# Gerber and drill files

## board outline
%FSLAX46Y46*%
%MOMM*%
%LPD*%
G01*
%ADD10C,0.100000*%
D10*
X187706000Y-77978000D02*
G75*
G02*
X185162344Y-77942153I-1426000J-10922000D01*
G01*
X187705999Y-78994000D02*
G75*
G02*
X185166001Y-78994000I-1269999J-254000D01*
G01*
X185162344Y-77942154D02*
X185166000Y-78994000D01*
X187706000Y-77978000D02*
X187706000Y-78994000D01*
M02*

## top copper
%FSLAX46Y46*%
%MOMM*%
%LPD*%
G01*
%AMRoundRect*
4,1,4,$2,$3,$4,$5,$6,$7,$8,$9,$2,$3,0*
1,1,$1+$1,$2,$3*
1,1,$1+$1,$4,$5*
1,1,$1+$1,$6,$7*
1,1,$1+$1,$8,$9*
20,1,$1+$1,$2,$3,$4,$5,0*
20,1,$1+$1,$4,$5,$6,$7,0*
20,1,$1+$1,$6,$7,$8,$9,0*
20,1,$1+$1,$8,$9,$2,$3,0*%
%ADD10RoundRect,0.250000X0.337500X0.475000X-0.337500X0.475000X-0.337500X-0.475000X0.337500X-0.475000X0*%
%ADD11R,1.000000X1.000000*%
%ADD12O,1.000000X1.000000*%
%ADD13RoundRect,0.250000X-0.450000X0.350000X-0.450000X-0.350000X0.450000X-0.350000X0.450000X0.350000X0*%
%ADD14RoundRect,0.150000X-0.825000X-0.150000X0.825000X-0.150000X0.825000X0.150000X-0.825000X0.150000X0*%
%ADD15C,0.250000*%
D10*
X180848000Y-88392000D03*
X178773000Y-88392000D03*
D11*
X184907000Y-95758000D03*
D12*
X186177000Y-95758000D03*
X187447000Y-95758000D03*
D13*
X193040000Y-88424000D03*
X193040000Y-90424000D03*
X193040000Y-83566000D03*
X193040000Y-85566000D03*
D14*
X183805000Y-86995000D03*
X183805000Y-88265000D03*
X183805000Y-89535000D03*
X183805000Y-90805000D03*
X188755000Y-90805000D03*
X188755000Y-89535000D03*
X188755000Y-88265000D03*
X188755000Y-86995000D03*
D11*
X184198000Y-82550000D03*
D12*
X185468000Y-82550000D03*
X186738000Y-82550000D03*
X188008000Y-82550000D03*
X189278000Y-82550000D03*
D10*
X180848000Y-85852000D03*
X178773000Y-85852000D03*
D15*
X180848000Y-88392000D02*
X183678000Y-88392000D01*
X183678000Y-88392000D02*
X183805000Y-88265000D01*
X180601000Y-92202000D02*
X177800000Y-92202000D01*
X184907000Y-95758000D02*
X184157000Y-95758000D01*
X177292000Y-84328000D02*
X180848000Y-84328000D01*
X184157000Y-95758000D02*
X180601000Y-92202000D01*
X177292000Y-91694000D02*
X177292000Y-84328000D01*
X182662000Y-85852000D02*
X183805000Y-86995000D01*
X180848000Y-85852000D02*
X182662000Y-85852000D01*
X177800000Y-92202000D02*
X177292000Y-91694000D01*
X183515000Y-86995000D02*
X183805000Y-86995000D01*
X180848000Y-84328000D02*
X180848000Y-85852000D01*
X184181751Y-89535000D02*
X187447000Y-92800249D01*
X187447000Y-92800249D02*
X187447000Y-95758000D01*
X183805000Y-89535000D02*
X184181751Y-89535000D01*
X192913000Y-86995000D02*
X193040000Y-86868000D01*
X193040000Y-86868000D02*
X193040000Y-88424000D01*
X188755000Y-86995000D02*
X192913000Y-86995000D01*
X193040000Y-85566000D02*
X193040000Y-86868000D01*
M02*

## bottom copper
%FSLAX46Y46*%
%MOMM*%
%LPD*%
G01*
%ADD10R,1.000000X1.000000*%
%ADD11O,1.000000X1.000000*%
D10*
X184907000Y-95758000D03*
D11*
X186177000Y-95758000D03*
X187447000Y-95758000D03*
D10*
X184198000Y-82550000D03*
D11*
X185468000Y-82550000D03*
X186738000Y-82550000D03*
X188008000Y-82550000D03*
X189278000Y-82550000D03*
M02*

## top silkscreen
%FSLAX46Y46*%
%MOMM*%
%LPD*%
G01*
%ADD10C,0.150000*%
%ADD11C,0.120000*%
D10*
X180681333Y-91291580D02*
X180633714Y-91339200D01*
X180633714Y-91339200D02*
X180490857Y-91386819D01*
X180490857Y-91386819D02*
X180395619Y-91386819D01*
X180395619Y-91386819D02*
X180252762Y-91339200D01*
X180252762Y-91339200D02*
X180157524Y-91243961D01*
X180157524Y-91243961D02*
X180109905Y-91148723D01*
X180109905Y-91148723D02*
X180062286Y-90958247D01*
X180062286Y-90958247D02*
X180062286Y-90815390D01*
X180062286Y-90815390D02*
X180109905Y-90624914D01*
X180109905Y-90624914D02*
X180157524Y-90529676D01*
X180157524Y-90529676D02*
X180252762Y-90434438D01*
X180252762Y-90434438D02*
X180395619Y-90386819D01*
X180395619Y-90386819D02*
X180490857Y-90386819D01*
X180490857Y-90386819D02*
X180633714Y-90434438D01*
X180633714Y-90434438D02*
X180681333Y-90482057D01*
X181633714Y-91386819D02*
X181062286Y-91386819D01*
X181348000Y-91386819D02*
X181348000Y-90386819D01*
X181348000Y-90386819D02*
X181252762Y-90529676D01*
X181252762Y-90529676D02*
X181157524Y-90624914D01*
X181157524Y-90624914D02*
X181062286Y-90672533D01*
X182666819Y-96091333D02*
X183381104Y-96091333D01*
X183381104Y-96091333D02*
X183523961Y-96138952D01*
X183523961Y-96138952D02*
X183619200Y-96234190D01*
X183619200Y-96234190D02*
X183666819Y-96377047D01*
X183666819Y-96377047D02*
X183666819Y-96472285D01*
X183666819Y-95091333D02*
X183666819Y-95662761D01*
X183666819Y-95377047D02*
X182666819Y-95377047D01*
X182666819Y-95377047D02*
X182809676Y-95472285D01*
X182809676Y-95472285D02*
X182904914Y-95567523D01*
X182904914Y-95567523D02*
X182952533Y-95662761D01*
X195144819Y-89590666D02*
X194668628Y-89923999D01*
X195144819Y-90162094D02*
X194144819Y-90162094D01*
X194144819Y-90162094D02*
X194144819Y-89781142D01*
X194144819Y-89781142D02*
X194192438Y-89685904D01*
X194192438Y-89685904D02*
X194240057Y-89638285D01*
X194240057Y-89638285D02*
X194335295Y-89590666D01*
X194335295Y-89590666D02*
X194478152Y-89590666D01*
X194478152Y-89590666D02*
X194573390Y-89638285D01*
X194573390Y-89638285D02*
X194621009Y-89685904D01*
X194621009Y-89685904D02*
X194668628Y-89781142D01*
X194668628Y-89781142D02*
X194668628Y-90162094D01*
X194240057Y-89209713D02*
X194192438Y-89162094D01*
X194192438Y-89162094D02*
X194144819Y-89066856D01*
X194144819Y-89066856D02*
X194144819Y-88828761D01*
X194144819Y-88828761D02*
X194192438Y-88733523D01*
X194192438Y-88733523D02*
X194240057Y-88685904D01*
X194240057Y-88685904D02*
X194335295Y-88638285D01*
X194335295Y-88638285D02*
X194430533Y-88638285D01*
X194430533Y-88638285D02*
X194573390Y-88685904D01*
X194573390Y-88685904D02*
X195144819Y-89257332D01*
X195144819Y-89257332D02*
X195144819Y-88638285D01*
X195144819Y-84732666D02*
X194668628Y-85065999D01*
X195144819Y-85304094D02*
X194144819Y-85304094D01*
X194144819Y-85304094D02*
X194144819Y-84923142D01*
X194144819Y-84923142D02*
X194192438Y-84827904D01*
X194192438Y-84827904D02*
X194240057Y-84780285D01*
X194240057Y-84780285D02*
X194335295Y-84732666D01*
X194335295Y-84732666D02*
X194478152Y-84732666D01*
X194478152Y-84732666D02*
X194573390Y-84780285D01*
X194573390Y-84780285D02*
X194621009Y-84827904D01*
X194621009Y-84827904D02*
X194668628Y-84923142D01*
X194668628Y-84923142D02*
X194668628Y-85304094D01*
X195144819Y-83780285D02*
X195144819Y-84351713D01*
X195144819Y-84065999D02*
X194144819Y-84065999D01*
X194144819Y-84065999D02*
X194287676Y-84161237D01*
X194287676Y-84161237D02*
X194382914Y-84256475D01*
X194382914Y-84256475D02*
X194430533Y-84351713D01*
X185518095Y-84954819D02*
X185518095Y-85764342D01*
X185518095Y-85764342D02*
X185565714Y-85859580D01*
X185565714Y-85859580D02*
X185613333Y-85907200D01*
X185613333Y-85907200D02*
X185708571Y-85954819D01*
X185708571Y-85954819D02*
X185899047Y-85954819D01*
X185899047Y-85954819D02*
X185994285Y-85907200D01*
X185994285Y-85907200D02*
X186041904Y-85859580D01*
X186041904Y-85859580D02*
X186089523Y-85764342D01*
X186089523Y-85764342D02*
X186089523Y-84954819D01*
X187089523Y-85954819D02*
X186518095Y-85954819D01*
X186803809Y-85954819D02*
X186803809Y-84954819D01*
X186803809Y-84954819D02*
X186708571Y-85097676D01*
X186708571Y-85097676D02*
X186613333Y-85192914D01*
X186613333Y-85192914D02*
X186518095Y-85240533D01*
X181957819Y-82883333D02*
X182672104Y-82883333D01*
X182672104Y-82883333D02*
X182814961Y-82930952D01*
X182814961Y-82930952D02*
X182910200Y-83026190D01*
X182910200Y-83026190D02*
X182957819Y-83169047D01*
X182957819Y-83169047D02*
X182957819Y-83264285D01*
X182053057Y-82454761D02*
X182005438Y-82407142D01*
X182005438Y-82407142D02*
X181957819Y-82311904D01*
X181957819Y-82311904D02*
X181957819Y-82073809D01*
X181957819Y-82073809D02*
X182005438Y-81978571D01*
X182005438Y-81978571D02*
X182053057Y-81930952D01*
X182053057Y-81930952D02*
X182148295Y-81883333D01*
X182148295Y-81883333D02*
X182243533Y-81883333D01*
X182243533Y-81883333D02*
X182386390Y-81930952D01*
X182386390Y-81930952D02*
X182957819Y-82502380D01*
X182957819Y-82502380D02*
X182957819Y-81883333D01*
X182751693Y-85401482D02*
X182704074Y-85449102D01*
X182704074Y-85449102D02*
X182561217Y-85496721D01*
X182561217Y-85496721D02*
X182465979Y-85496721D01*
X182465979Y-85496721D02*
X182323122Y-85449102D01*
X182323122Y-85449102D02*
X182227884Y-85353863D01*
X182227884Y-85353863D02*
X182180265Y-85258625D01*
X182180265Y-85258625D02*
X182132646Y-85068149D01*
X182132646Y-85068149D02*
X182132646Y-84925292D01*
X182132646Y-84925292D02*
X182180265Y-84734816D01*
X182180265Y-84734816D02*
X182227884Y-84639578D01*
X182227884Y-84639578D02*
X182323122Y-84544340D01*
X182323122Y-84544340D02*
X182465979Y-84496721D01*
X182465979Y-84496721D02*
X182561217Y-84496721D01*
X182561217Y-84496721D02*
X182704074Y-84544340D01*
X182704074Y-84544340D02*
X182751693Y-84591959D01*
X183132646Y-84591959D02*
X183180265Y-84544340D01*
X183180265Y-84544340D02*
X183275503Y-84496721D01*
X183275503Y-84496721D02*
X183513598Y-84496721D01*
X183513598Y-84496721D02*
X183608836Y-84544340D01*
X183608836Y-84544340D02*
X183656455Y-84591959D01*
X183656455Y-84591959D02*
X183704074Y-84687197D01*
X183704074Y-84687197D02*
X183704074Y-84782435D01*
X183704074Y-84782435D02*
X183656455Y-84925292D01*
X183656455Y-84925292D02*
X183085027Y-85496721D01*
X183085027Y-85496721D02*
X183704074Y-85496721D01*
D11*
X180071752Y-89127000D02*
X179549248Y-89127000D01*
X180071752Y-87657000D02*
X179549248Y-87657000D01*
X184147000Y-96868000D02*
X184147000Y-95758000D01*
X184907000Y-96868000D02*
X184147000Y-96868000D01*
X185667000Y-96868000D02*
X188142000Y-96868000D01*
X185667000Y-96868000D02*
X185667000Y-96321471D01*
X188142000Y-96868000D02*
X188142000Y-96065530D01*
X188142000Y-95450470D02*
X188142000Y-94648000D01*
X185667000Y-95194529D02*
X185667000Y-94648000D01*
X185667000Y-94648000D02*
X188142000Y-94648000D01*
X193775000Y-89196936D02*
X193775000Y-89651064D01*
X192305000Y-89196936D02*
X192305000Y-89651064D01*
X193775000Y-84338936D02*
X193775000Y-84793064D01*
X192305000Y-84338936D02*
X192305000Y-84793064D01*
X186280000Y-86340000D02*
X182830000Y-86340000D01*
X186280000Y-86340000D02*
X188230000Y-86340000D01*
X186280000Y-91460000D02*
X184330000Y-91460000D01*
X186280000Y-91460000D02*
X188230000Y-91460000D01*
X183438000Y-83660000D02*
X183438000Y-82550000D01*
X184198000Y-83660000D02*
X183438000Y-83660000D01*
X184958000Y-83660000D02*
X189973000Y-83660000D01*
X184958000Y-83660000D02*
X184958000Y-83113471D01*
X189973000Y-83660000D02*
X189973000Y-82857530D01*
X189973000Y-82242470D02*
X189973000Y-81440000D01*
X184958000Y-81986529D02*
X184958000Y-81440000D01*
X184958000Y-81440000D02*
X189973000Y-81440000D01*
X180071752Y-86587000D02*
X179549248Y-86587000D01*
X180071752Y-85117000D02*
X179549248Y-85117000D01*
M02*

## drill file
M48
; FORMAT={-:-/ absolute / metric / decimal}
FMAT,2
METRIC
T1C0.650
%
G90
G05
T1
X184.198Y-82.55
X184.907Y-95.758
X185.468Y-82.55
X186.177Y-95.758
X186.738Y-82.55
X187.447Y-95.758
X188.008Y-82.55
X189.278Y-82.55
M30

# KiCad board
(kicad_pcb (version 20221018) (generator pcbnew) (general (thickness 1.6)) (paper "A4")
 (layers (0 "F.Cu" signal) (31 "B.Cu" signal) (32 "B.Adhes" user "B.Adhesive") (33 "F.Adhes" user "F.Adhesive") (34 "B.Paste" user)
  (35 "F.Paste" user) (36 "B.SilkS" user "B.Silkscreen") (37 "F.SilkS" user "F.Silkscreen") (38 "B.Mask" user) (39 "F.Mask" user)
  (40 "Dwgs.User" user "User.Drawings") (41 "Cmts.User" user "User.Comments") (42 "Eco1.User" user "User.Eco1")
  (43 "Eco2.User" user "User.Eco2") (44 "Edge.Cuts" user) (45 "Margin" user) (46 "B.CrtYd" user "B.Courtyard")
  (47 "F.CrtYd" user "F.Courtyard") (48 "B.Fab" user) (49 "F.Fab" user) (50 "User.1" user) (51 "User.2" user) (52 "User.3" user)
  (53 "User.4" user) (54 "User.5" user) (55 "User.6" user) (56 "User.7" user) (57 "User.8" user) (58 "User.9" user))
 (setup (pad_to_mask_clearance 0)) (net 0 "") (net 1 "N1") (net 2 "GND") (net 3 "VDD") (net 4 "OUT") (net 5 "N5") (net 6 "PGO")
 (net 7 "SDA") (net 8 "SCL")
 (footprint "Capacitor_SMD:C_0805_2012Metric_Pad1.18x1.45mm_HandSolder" (layer "F.Cu") (at 179.8105 88.392 180)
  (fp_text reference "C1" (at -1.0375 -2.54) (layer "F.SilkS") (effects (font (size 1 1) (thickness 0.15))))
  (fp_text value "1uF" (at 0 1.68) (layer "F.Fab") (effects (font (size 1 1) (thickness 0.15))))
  (fp_line (start -0.261252 -0.735) (end 0.261252 -0.735) (stroke (width 0.12) (type solid)) (layer "F.SilkS"))
  (fp_line (start -0.261252 0.735) (end 0.261252 0.735) (stroke (width 0.12) (type solid)) (layer "F.SilkS"))
  (pad "1" smd roundrect (at -1.0375 0 180) (size 1.175 1.45) (layers "F.Cu" "F.Paste" "F.Mask") (roundrect_rratio 0.212766) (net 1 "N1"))
  (pad "2" smd roundrect (at 1.0375 0 180) (size 1.175 1.45) (layers "F.Cu" "F.Paste" "F.Mask") (roundrect_rratio 0.212766) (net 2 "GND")))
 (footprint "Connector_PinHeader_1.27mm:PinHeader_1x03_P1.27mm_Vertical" (layer "F.Cu") (at 184.907 95.758 90)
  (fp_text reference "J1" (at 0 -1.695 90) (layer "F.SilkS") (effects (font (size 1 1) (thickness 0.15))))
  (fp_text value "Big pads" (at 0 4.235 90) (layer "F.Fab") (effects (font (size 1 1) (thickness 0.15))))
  (fp_line (start -1.11 -0.76) (end 0 -0.76) (stroke (width 0.12) (type solid)) (layer "F.SilkS"))
  (fp_line (start -1.11 0) (end -1.11 -0.76) (stroke (width 0.12) (type solid)) (layer "F.SilkS"))
  (fp_line (start -1.11 0.76) (end -1.11 3.235) (stroke (width 0.12) (type solid)) (layer "F.SilkS"))
  (fp_line (start -1.11 0.76) (end -0.563471 0.76) (stroke (width 0.12) (type solid)) (layer "F.SilkS"))
  (fp_line (start -1.11 3.235) (end -0.30753 3.235) (stroke (width 0.12) (type solid)) (layer "F.SilkS"))
  (fp_line (start 0.30753 3.235) (end 1.11 3.235) (stroke (width 0.12) (type solid)) (layer "F.SilkS"))
  (fp_line (start 0.563471 0.76) (end 1.11 0.76) (stroke (width 0.12) (type solid)) (layer "F.SilkS"))
  (fp_line (start 1.11 0.76) (end 1.11 3.235) (stroke (width 0.12) (type solid)) (layer "F.SilkS"))
  (pad "1" thru_hole rect (at 0 0 90) (size 1 1) (drill 0.65) (layers "*.Cu" "*.Mask") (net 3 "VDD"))
  (pad "2" thru_hole oval (at 0 1.27 90) (size 1 1) (drill 0.65) (layers "*.Cu" "*.Mask") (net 2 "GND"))
  (pad "3" thru_hole oval (at 0 2.54 90) (size 1 1) (drill 0.65) (layers "*.Cu" "*.Mask") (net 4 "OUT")))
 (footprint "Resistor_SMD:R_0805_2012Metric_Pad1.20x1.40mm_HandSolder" (layer "F.Cu") (at 193.04 89.424 -90)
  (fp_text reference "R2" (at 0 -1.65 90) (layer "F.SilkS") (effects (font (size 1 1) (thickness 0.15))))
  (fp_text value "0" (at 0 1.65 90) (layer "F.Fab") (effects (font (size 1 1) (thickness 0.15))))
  (fp_line (start -0.227064 -0.735) (end 0.227064 -0.735) (stroke (width 0.12) (type solid)) (layer "F.SilkS"))
  (fp_line (start -0.227064 0.735) (end 0.227064 0.735) (stroke (width 0.12) (type solid)) (layer "F.SilkS"))
  (pad "1" smd roundrect (at -1 0 270) (size 1.2 1.4) (layers "F.Cu" "F.Paste" "F.Mask") (roundrect_rratio 0.208333) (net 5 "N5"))
  (pad "2" smd roundrect (at 1 0 270) (size 1.2 1.4) (layers "F.Cu" "F.Paste" "F.Mask") (roundrect_rratio 0.208333) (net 2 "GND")))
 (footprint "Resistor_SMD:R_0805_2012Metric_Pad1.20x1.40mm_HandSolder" (layer "F.Cu") (at 193.04 84.566 -90)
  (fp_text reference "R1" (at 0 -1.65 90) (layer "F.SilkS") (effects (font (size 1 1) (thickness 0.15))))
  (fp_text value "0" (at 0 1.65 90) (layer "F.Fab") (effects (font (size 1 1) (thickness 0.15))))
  (fp_line (start -0.227064 -0.735) (end 0.227064 -0.735) (stroke (width 0.12) (type solid)) (layer "F.SilkS"))
  (fp_line (start -0.227064 0.735) (end 0.227064 0.735) (stroke (width 0.12) (type solid)) (layer "F.SilkS"))
  (pad "1" smd roundrect (at -1 0 270) (size 1.2 1.4) (layers "F.Cu" "F.Paste" "F.Mask") (roundrect_rratio 0.208333) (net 3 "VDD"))
  (pad "2" smd roundrect (at 1 0 270) (size 1.2 1.4) (layers "F.Cu" "F.Paste" "F.Mask") (roundrect_rratio 0.208333) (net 5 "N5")))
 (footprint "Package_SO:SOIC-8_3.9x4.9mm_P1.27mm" (layer "F.Cu") (at 186.28 88.9)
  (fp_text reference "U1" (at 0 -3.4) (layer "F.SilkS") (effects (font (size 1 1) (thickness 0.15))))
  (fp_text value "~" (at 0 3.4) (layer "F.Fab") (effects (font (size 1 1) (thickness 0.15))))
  (fp_line (start 0 -2.56) (end -3.45 -2.56) (stroke (width 0.12) (type solid)) (layer "F.SilkS"))
  (fp_line (start 0 -2.56) (end 1.95 -2.56) (stroke (width 0.12) (type solid)) (layer "F.SilkS"))
  (fp_line (start 0 2.56) (end -1.95 2.56) (stroke (width 0.12) (type solid)) (layer "F.SilkS"))
  (fp_line (start 0 2.56) (end 1.95 2.56) (stroke (width 0.12) (type solid)) (layer "F.SilkS"))
  (pad "1" smd roundrect (at -2.475 -1.905) (size 1.95 0.6) (layers "F.Cu" "F.Paste" "F.Mask") (roundrect_rratio 0.25) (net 3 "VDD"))
  (pad "2" smd roundrect (at -2.475 -0.635) (size 1.95 0.6) (layers "F.Cu" "F.Paste" "F.Mask") (roundrect_rratio 0.25) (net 1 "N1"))
  (pad "3" smd roundrect (at -2.475 0.635) (size 1.95 0.6) (layers "F.Cu" "F.Paste" "F.Mask") (roundrect_rratio 0.25) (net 4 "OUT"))
  (pad "4" smd roundrect (at -2.475 1.905) (size 1.95 0.6) (layers "F.Cu" "F.Paste" "F.Mask") (roundrect_rratio 0.25) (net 2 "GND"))
  (pad "5" smd roundrect (at 2.475 1.905) (size 1.95 0.6) (layers "F.Cu" "F.Paste" "F.Mask") (roundrect_rratio 0.25) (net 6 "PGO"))
  (pad "6" smd roundrect (at 2.475 0.635) (size 1.95 0.6) (layers "F.Cu" "F.Paste" "F.Mask") (roundrect_rratio 0.25) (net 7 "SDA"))
  (pad "7" smd roundrect (at 2.475 -0.635) (size 1.95 0.6) (layers "F.Cu" "F.Paste" "F.Mask") (roundrect_rratio 0.25) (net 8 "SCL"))
  (pad "8" smd roundrect (at 2.475 -1.905) (size 1.95 0.6) (layers "F.Cu" "F.Paste" "F.Mask") (roundrect_rratio 0.25) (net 5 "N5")))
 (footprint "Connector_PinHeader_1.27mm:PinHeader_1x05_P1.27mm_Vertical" (layer "F.Cu") (at 184.198 82.55 90)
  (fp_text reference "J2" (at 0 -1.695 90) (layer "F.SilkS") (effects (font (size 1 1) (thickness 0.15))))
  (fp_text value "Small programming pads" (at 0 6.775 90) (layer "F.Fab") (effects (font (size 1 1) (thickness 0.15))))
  (fp_line (start -1.11 -0.76) (end 0 -0.76) (stroke (width 0.12) (type solid)) (layer "F.SilkS"))
  (fp_line (start -1.11 0) (end -1.11 -0.76) (stroke (width 0.12) (type solid)) (layer "F.SilkS"))
  (fp_line (start -1.11 0.76) (end -1.11 5.775) (stroke (width 0.12) (type solid)) (layer "F.SilkS"))
  (fp_line (start -1.11 0.76) (end -0.563471 0.76) (stroke (width 0.12) (type solid)) (layer "F.SilkS"))
  (fp_line (start -1.11 5.775) (end -0.30753 5.775) (stroke (width 0.12) (type solid)) (layer "F.SilkS"))
  (fp_line (start 0.30753 5.775) (end 1.11 5.775) (stroke (width 0.12) (type solid)) (layer "F.SilkS"))
  (fp_line (start 0.563471 0.76) (end 1.11 0.76) (stroke (width 0.12) (type solid)) (layer "F.SilkS"))
  (fp_line (start 1.11 0.76) (end 1.11 5.775) (stroke (width 0.12) (type solid)) (layer "F.SilkS"))
  (pad "1" thru_hole rect (at 0 0 90) (size 1 1) (drill 0.65) (layers "*.Cu" "*.Mask") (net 3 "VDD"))
  (pad "2" thru_hole oval (at 0 1.27 90) (size 1 1) (drill 0.65) (layers "*.Cu" "*.Mask") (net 6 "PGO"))
  (pad "3" thru_hole oval (at 0 2.54 90) (size 1 1) (drill 0.65) (layers "*.Cu" "*.Mask") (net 8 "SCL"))
  (pad "4" thru_hole oval (at 0 3.81 90) (size 1 1) (drill 0.65) (layers "*.Cu" "*.Mask") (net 7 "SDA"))
  (pad "5" thru_hole oval (at 0 5.08 90) (size 1 1) (drill 0.65) (layers "*.Cu" "*.Mask") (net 2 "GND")))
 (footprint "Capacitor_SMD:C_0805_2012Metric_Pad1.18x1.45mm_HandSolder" (layer "F.Cu") (at 179.8105 85.852 180)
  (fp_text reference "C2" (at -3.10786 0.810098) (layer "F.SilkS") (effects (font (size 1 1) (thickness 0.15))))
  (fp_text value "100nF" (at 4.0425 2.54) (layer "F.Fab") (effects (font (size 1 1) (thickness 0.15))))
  (fp_line (start -0.261252 -0.735) (end 0.261252 -0.735) (stroke (width 0.12) (type solid)) (layer "F.SilkS"))
  (fp_line (start -0.261252 0.735) (end 0.261252 0.735) (stroke (width 0.12) (type solid)) (layer "F.SilkS"))
  (pad "1" smd roundrect (at -1.0375 0 180) (size 1.175 1.45) (layers "F.Cu" "F.Paste" "F.Mask") (roundrect_rratio 0.212766) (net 3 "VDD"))
  (pad "2" smd roundrect (at 1.0375 0 180) (size 1.175 1.45) (layers "F.Cu" "F.Paste" "F.Mask") (roundrect_rratio 0.212766) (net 2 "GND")))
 (gr_arc (start 187.706 77.978) (mid 186.12479 99.913604) (end 185.162344 77.942154) (stroke (width 0.1) (type default)) (layer "Edge.Cuts"))
 (gr_arc (start 187.705999 78.994) (mid 186.436 80.54315) (end 185.166001 78.994) (stroke (width 0.1) (type default)) (layer "Edge.Cuts"))
 (gr_line (start 185.162344 77.942154) (end 185.166 78.994) (stroke (width 0.1) (type default)) (layer "Edge.Cuts"))
 (gr_line (start 187.706 77.978) (end 187.706 78.994) (stroke (width 0.1) (type default)) (layer "Edge.Cuts"))
 (segment (start 180.848 88.392) (end 183.678 88.392) (width 0.25) (layer "F.Cu") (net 1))
 (segment (start 183.678 88.392) (end 183.805 88.265) (width 0.25) (layer "F.Cu") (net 1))
 (segment (start 180.601 92.202) (end 177.8 92.202) (width 0.25) (layer "F.Cu") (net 3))
 (segment (start 184.907 95.758) (end 184.157 95.758) (width 0.25) (layer "F.Cu") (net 3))
 (segment (start 177.292 84.328) (end 180.848 84.328) (width 0.25) (layer "F.Cu") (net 3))
 (segment (start 184.157 95.758) (end 180.601 92.202) (width 0.25) (layer "F.Cu") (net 3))
 (segment (start 177.292 91.694) (end 177.292 84.328) (width 0.25) (layer "F.Cu") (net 3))
 (segment (start 182.662 85.852) (end 183.805 86.995) (width 0.25) (layer "F.Cu") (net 3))
 (segment (start 180.848 85.852) (end 182.662 85.852) (width 0.25) (layer "F.Cu") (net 3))
 (segment (start 177.8 92.202) (end 177.292 91.694) (width 0.25) (layer "F.Cu") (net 3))
 (segment (start 183.515 86.995) (end 183.805 86.995) (width 0.25) (layer "F.Cu") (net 3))
 (segment (start 180.848 84.328) (end 180.848 85.852) (width 0.25) (layer "F.Cu") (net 3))
 (segment (start 184.181751 89.535) (end 187.447 92.800249) (width 0.25) (layer "F.Cu") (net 4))
 (segment (start 187.447 92.800249) (end 187.447 95.758) (width 0.25) (layer "F.Cu") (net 4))
 (segment (start 183.805 89.535) (end 184.181751 89.535) (width 0.25) (layer "F.Cu") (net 4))
 (segment (start 192.913 86.995) (end 193.04 86.868) (width 0.25) (layer "F.Cu") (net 5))
 (segment (start 193.04 86.868) (end 193.04 88.424) (width 0.25) (layer "F.Cu") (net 5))
 (segment (start 188.755 86.995) (end 192.913 86.995) (width 0.25) (layer "F.Cu") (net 5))
 (segment (start 193.04 85.566) (end 193.04 86.868) (width 0.25) (layer "F.Cu") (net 5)))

